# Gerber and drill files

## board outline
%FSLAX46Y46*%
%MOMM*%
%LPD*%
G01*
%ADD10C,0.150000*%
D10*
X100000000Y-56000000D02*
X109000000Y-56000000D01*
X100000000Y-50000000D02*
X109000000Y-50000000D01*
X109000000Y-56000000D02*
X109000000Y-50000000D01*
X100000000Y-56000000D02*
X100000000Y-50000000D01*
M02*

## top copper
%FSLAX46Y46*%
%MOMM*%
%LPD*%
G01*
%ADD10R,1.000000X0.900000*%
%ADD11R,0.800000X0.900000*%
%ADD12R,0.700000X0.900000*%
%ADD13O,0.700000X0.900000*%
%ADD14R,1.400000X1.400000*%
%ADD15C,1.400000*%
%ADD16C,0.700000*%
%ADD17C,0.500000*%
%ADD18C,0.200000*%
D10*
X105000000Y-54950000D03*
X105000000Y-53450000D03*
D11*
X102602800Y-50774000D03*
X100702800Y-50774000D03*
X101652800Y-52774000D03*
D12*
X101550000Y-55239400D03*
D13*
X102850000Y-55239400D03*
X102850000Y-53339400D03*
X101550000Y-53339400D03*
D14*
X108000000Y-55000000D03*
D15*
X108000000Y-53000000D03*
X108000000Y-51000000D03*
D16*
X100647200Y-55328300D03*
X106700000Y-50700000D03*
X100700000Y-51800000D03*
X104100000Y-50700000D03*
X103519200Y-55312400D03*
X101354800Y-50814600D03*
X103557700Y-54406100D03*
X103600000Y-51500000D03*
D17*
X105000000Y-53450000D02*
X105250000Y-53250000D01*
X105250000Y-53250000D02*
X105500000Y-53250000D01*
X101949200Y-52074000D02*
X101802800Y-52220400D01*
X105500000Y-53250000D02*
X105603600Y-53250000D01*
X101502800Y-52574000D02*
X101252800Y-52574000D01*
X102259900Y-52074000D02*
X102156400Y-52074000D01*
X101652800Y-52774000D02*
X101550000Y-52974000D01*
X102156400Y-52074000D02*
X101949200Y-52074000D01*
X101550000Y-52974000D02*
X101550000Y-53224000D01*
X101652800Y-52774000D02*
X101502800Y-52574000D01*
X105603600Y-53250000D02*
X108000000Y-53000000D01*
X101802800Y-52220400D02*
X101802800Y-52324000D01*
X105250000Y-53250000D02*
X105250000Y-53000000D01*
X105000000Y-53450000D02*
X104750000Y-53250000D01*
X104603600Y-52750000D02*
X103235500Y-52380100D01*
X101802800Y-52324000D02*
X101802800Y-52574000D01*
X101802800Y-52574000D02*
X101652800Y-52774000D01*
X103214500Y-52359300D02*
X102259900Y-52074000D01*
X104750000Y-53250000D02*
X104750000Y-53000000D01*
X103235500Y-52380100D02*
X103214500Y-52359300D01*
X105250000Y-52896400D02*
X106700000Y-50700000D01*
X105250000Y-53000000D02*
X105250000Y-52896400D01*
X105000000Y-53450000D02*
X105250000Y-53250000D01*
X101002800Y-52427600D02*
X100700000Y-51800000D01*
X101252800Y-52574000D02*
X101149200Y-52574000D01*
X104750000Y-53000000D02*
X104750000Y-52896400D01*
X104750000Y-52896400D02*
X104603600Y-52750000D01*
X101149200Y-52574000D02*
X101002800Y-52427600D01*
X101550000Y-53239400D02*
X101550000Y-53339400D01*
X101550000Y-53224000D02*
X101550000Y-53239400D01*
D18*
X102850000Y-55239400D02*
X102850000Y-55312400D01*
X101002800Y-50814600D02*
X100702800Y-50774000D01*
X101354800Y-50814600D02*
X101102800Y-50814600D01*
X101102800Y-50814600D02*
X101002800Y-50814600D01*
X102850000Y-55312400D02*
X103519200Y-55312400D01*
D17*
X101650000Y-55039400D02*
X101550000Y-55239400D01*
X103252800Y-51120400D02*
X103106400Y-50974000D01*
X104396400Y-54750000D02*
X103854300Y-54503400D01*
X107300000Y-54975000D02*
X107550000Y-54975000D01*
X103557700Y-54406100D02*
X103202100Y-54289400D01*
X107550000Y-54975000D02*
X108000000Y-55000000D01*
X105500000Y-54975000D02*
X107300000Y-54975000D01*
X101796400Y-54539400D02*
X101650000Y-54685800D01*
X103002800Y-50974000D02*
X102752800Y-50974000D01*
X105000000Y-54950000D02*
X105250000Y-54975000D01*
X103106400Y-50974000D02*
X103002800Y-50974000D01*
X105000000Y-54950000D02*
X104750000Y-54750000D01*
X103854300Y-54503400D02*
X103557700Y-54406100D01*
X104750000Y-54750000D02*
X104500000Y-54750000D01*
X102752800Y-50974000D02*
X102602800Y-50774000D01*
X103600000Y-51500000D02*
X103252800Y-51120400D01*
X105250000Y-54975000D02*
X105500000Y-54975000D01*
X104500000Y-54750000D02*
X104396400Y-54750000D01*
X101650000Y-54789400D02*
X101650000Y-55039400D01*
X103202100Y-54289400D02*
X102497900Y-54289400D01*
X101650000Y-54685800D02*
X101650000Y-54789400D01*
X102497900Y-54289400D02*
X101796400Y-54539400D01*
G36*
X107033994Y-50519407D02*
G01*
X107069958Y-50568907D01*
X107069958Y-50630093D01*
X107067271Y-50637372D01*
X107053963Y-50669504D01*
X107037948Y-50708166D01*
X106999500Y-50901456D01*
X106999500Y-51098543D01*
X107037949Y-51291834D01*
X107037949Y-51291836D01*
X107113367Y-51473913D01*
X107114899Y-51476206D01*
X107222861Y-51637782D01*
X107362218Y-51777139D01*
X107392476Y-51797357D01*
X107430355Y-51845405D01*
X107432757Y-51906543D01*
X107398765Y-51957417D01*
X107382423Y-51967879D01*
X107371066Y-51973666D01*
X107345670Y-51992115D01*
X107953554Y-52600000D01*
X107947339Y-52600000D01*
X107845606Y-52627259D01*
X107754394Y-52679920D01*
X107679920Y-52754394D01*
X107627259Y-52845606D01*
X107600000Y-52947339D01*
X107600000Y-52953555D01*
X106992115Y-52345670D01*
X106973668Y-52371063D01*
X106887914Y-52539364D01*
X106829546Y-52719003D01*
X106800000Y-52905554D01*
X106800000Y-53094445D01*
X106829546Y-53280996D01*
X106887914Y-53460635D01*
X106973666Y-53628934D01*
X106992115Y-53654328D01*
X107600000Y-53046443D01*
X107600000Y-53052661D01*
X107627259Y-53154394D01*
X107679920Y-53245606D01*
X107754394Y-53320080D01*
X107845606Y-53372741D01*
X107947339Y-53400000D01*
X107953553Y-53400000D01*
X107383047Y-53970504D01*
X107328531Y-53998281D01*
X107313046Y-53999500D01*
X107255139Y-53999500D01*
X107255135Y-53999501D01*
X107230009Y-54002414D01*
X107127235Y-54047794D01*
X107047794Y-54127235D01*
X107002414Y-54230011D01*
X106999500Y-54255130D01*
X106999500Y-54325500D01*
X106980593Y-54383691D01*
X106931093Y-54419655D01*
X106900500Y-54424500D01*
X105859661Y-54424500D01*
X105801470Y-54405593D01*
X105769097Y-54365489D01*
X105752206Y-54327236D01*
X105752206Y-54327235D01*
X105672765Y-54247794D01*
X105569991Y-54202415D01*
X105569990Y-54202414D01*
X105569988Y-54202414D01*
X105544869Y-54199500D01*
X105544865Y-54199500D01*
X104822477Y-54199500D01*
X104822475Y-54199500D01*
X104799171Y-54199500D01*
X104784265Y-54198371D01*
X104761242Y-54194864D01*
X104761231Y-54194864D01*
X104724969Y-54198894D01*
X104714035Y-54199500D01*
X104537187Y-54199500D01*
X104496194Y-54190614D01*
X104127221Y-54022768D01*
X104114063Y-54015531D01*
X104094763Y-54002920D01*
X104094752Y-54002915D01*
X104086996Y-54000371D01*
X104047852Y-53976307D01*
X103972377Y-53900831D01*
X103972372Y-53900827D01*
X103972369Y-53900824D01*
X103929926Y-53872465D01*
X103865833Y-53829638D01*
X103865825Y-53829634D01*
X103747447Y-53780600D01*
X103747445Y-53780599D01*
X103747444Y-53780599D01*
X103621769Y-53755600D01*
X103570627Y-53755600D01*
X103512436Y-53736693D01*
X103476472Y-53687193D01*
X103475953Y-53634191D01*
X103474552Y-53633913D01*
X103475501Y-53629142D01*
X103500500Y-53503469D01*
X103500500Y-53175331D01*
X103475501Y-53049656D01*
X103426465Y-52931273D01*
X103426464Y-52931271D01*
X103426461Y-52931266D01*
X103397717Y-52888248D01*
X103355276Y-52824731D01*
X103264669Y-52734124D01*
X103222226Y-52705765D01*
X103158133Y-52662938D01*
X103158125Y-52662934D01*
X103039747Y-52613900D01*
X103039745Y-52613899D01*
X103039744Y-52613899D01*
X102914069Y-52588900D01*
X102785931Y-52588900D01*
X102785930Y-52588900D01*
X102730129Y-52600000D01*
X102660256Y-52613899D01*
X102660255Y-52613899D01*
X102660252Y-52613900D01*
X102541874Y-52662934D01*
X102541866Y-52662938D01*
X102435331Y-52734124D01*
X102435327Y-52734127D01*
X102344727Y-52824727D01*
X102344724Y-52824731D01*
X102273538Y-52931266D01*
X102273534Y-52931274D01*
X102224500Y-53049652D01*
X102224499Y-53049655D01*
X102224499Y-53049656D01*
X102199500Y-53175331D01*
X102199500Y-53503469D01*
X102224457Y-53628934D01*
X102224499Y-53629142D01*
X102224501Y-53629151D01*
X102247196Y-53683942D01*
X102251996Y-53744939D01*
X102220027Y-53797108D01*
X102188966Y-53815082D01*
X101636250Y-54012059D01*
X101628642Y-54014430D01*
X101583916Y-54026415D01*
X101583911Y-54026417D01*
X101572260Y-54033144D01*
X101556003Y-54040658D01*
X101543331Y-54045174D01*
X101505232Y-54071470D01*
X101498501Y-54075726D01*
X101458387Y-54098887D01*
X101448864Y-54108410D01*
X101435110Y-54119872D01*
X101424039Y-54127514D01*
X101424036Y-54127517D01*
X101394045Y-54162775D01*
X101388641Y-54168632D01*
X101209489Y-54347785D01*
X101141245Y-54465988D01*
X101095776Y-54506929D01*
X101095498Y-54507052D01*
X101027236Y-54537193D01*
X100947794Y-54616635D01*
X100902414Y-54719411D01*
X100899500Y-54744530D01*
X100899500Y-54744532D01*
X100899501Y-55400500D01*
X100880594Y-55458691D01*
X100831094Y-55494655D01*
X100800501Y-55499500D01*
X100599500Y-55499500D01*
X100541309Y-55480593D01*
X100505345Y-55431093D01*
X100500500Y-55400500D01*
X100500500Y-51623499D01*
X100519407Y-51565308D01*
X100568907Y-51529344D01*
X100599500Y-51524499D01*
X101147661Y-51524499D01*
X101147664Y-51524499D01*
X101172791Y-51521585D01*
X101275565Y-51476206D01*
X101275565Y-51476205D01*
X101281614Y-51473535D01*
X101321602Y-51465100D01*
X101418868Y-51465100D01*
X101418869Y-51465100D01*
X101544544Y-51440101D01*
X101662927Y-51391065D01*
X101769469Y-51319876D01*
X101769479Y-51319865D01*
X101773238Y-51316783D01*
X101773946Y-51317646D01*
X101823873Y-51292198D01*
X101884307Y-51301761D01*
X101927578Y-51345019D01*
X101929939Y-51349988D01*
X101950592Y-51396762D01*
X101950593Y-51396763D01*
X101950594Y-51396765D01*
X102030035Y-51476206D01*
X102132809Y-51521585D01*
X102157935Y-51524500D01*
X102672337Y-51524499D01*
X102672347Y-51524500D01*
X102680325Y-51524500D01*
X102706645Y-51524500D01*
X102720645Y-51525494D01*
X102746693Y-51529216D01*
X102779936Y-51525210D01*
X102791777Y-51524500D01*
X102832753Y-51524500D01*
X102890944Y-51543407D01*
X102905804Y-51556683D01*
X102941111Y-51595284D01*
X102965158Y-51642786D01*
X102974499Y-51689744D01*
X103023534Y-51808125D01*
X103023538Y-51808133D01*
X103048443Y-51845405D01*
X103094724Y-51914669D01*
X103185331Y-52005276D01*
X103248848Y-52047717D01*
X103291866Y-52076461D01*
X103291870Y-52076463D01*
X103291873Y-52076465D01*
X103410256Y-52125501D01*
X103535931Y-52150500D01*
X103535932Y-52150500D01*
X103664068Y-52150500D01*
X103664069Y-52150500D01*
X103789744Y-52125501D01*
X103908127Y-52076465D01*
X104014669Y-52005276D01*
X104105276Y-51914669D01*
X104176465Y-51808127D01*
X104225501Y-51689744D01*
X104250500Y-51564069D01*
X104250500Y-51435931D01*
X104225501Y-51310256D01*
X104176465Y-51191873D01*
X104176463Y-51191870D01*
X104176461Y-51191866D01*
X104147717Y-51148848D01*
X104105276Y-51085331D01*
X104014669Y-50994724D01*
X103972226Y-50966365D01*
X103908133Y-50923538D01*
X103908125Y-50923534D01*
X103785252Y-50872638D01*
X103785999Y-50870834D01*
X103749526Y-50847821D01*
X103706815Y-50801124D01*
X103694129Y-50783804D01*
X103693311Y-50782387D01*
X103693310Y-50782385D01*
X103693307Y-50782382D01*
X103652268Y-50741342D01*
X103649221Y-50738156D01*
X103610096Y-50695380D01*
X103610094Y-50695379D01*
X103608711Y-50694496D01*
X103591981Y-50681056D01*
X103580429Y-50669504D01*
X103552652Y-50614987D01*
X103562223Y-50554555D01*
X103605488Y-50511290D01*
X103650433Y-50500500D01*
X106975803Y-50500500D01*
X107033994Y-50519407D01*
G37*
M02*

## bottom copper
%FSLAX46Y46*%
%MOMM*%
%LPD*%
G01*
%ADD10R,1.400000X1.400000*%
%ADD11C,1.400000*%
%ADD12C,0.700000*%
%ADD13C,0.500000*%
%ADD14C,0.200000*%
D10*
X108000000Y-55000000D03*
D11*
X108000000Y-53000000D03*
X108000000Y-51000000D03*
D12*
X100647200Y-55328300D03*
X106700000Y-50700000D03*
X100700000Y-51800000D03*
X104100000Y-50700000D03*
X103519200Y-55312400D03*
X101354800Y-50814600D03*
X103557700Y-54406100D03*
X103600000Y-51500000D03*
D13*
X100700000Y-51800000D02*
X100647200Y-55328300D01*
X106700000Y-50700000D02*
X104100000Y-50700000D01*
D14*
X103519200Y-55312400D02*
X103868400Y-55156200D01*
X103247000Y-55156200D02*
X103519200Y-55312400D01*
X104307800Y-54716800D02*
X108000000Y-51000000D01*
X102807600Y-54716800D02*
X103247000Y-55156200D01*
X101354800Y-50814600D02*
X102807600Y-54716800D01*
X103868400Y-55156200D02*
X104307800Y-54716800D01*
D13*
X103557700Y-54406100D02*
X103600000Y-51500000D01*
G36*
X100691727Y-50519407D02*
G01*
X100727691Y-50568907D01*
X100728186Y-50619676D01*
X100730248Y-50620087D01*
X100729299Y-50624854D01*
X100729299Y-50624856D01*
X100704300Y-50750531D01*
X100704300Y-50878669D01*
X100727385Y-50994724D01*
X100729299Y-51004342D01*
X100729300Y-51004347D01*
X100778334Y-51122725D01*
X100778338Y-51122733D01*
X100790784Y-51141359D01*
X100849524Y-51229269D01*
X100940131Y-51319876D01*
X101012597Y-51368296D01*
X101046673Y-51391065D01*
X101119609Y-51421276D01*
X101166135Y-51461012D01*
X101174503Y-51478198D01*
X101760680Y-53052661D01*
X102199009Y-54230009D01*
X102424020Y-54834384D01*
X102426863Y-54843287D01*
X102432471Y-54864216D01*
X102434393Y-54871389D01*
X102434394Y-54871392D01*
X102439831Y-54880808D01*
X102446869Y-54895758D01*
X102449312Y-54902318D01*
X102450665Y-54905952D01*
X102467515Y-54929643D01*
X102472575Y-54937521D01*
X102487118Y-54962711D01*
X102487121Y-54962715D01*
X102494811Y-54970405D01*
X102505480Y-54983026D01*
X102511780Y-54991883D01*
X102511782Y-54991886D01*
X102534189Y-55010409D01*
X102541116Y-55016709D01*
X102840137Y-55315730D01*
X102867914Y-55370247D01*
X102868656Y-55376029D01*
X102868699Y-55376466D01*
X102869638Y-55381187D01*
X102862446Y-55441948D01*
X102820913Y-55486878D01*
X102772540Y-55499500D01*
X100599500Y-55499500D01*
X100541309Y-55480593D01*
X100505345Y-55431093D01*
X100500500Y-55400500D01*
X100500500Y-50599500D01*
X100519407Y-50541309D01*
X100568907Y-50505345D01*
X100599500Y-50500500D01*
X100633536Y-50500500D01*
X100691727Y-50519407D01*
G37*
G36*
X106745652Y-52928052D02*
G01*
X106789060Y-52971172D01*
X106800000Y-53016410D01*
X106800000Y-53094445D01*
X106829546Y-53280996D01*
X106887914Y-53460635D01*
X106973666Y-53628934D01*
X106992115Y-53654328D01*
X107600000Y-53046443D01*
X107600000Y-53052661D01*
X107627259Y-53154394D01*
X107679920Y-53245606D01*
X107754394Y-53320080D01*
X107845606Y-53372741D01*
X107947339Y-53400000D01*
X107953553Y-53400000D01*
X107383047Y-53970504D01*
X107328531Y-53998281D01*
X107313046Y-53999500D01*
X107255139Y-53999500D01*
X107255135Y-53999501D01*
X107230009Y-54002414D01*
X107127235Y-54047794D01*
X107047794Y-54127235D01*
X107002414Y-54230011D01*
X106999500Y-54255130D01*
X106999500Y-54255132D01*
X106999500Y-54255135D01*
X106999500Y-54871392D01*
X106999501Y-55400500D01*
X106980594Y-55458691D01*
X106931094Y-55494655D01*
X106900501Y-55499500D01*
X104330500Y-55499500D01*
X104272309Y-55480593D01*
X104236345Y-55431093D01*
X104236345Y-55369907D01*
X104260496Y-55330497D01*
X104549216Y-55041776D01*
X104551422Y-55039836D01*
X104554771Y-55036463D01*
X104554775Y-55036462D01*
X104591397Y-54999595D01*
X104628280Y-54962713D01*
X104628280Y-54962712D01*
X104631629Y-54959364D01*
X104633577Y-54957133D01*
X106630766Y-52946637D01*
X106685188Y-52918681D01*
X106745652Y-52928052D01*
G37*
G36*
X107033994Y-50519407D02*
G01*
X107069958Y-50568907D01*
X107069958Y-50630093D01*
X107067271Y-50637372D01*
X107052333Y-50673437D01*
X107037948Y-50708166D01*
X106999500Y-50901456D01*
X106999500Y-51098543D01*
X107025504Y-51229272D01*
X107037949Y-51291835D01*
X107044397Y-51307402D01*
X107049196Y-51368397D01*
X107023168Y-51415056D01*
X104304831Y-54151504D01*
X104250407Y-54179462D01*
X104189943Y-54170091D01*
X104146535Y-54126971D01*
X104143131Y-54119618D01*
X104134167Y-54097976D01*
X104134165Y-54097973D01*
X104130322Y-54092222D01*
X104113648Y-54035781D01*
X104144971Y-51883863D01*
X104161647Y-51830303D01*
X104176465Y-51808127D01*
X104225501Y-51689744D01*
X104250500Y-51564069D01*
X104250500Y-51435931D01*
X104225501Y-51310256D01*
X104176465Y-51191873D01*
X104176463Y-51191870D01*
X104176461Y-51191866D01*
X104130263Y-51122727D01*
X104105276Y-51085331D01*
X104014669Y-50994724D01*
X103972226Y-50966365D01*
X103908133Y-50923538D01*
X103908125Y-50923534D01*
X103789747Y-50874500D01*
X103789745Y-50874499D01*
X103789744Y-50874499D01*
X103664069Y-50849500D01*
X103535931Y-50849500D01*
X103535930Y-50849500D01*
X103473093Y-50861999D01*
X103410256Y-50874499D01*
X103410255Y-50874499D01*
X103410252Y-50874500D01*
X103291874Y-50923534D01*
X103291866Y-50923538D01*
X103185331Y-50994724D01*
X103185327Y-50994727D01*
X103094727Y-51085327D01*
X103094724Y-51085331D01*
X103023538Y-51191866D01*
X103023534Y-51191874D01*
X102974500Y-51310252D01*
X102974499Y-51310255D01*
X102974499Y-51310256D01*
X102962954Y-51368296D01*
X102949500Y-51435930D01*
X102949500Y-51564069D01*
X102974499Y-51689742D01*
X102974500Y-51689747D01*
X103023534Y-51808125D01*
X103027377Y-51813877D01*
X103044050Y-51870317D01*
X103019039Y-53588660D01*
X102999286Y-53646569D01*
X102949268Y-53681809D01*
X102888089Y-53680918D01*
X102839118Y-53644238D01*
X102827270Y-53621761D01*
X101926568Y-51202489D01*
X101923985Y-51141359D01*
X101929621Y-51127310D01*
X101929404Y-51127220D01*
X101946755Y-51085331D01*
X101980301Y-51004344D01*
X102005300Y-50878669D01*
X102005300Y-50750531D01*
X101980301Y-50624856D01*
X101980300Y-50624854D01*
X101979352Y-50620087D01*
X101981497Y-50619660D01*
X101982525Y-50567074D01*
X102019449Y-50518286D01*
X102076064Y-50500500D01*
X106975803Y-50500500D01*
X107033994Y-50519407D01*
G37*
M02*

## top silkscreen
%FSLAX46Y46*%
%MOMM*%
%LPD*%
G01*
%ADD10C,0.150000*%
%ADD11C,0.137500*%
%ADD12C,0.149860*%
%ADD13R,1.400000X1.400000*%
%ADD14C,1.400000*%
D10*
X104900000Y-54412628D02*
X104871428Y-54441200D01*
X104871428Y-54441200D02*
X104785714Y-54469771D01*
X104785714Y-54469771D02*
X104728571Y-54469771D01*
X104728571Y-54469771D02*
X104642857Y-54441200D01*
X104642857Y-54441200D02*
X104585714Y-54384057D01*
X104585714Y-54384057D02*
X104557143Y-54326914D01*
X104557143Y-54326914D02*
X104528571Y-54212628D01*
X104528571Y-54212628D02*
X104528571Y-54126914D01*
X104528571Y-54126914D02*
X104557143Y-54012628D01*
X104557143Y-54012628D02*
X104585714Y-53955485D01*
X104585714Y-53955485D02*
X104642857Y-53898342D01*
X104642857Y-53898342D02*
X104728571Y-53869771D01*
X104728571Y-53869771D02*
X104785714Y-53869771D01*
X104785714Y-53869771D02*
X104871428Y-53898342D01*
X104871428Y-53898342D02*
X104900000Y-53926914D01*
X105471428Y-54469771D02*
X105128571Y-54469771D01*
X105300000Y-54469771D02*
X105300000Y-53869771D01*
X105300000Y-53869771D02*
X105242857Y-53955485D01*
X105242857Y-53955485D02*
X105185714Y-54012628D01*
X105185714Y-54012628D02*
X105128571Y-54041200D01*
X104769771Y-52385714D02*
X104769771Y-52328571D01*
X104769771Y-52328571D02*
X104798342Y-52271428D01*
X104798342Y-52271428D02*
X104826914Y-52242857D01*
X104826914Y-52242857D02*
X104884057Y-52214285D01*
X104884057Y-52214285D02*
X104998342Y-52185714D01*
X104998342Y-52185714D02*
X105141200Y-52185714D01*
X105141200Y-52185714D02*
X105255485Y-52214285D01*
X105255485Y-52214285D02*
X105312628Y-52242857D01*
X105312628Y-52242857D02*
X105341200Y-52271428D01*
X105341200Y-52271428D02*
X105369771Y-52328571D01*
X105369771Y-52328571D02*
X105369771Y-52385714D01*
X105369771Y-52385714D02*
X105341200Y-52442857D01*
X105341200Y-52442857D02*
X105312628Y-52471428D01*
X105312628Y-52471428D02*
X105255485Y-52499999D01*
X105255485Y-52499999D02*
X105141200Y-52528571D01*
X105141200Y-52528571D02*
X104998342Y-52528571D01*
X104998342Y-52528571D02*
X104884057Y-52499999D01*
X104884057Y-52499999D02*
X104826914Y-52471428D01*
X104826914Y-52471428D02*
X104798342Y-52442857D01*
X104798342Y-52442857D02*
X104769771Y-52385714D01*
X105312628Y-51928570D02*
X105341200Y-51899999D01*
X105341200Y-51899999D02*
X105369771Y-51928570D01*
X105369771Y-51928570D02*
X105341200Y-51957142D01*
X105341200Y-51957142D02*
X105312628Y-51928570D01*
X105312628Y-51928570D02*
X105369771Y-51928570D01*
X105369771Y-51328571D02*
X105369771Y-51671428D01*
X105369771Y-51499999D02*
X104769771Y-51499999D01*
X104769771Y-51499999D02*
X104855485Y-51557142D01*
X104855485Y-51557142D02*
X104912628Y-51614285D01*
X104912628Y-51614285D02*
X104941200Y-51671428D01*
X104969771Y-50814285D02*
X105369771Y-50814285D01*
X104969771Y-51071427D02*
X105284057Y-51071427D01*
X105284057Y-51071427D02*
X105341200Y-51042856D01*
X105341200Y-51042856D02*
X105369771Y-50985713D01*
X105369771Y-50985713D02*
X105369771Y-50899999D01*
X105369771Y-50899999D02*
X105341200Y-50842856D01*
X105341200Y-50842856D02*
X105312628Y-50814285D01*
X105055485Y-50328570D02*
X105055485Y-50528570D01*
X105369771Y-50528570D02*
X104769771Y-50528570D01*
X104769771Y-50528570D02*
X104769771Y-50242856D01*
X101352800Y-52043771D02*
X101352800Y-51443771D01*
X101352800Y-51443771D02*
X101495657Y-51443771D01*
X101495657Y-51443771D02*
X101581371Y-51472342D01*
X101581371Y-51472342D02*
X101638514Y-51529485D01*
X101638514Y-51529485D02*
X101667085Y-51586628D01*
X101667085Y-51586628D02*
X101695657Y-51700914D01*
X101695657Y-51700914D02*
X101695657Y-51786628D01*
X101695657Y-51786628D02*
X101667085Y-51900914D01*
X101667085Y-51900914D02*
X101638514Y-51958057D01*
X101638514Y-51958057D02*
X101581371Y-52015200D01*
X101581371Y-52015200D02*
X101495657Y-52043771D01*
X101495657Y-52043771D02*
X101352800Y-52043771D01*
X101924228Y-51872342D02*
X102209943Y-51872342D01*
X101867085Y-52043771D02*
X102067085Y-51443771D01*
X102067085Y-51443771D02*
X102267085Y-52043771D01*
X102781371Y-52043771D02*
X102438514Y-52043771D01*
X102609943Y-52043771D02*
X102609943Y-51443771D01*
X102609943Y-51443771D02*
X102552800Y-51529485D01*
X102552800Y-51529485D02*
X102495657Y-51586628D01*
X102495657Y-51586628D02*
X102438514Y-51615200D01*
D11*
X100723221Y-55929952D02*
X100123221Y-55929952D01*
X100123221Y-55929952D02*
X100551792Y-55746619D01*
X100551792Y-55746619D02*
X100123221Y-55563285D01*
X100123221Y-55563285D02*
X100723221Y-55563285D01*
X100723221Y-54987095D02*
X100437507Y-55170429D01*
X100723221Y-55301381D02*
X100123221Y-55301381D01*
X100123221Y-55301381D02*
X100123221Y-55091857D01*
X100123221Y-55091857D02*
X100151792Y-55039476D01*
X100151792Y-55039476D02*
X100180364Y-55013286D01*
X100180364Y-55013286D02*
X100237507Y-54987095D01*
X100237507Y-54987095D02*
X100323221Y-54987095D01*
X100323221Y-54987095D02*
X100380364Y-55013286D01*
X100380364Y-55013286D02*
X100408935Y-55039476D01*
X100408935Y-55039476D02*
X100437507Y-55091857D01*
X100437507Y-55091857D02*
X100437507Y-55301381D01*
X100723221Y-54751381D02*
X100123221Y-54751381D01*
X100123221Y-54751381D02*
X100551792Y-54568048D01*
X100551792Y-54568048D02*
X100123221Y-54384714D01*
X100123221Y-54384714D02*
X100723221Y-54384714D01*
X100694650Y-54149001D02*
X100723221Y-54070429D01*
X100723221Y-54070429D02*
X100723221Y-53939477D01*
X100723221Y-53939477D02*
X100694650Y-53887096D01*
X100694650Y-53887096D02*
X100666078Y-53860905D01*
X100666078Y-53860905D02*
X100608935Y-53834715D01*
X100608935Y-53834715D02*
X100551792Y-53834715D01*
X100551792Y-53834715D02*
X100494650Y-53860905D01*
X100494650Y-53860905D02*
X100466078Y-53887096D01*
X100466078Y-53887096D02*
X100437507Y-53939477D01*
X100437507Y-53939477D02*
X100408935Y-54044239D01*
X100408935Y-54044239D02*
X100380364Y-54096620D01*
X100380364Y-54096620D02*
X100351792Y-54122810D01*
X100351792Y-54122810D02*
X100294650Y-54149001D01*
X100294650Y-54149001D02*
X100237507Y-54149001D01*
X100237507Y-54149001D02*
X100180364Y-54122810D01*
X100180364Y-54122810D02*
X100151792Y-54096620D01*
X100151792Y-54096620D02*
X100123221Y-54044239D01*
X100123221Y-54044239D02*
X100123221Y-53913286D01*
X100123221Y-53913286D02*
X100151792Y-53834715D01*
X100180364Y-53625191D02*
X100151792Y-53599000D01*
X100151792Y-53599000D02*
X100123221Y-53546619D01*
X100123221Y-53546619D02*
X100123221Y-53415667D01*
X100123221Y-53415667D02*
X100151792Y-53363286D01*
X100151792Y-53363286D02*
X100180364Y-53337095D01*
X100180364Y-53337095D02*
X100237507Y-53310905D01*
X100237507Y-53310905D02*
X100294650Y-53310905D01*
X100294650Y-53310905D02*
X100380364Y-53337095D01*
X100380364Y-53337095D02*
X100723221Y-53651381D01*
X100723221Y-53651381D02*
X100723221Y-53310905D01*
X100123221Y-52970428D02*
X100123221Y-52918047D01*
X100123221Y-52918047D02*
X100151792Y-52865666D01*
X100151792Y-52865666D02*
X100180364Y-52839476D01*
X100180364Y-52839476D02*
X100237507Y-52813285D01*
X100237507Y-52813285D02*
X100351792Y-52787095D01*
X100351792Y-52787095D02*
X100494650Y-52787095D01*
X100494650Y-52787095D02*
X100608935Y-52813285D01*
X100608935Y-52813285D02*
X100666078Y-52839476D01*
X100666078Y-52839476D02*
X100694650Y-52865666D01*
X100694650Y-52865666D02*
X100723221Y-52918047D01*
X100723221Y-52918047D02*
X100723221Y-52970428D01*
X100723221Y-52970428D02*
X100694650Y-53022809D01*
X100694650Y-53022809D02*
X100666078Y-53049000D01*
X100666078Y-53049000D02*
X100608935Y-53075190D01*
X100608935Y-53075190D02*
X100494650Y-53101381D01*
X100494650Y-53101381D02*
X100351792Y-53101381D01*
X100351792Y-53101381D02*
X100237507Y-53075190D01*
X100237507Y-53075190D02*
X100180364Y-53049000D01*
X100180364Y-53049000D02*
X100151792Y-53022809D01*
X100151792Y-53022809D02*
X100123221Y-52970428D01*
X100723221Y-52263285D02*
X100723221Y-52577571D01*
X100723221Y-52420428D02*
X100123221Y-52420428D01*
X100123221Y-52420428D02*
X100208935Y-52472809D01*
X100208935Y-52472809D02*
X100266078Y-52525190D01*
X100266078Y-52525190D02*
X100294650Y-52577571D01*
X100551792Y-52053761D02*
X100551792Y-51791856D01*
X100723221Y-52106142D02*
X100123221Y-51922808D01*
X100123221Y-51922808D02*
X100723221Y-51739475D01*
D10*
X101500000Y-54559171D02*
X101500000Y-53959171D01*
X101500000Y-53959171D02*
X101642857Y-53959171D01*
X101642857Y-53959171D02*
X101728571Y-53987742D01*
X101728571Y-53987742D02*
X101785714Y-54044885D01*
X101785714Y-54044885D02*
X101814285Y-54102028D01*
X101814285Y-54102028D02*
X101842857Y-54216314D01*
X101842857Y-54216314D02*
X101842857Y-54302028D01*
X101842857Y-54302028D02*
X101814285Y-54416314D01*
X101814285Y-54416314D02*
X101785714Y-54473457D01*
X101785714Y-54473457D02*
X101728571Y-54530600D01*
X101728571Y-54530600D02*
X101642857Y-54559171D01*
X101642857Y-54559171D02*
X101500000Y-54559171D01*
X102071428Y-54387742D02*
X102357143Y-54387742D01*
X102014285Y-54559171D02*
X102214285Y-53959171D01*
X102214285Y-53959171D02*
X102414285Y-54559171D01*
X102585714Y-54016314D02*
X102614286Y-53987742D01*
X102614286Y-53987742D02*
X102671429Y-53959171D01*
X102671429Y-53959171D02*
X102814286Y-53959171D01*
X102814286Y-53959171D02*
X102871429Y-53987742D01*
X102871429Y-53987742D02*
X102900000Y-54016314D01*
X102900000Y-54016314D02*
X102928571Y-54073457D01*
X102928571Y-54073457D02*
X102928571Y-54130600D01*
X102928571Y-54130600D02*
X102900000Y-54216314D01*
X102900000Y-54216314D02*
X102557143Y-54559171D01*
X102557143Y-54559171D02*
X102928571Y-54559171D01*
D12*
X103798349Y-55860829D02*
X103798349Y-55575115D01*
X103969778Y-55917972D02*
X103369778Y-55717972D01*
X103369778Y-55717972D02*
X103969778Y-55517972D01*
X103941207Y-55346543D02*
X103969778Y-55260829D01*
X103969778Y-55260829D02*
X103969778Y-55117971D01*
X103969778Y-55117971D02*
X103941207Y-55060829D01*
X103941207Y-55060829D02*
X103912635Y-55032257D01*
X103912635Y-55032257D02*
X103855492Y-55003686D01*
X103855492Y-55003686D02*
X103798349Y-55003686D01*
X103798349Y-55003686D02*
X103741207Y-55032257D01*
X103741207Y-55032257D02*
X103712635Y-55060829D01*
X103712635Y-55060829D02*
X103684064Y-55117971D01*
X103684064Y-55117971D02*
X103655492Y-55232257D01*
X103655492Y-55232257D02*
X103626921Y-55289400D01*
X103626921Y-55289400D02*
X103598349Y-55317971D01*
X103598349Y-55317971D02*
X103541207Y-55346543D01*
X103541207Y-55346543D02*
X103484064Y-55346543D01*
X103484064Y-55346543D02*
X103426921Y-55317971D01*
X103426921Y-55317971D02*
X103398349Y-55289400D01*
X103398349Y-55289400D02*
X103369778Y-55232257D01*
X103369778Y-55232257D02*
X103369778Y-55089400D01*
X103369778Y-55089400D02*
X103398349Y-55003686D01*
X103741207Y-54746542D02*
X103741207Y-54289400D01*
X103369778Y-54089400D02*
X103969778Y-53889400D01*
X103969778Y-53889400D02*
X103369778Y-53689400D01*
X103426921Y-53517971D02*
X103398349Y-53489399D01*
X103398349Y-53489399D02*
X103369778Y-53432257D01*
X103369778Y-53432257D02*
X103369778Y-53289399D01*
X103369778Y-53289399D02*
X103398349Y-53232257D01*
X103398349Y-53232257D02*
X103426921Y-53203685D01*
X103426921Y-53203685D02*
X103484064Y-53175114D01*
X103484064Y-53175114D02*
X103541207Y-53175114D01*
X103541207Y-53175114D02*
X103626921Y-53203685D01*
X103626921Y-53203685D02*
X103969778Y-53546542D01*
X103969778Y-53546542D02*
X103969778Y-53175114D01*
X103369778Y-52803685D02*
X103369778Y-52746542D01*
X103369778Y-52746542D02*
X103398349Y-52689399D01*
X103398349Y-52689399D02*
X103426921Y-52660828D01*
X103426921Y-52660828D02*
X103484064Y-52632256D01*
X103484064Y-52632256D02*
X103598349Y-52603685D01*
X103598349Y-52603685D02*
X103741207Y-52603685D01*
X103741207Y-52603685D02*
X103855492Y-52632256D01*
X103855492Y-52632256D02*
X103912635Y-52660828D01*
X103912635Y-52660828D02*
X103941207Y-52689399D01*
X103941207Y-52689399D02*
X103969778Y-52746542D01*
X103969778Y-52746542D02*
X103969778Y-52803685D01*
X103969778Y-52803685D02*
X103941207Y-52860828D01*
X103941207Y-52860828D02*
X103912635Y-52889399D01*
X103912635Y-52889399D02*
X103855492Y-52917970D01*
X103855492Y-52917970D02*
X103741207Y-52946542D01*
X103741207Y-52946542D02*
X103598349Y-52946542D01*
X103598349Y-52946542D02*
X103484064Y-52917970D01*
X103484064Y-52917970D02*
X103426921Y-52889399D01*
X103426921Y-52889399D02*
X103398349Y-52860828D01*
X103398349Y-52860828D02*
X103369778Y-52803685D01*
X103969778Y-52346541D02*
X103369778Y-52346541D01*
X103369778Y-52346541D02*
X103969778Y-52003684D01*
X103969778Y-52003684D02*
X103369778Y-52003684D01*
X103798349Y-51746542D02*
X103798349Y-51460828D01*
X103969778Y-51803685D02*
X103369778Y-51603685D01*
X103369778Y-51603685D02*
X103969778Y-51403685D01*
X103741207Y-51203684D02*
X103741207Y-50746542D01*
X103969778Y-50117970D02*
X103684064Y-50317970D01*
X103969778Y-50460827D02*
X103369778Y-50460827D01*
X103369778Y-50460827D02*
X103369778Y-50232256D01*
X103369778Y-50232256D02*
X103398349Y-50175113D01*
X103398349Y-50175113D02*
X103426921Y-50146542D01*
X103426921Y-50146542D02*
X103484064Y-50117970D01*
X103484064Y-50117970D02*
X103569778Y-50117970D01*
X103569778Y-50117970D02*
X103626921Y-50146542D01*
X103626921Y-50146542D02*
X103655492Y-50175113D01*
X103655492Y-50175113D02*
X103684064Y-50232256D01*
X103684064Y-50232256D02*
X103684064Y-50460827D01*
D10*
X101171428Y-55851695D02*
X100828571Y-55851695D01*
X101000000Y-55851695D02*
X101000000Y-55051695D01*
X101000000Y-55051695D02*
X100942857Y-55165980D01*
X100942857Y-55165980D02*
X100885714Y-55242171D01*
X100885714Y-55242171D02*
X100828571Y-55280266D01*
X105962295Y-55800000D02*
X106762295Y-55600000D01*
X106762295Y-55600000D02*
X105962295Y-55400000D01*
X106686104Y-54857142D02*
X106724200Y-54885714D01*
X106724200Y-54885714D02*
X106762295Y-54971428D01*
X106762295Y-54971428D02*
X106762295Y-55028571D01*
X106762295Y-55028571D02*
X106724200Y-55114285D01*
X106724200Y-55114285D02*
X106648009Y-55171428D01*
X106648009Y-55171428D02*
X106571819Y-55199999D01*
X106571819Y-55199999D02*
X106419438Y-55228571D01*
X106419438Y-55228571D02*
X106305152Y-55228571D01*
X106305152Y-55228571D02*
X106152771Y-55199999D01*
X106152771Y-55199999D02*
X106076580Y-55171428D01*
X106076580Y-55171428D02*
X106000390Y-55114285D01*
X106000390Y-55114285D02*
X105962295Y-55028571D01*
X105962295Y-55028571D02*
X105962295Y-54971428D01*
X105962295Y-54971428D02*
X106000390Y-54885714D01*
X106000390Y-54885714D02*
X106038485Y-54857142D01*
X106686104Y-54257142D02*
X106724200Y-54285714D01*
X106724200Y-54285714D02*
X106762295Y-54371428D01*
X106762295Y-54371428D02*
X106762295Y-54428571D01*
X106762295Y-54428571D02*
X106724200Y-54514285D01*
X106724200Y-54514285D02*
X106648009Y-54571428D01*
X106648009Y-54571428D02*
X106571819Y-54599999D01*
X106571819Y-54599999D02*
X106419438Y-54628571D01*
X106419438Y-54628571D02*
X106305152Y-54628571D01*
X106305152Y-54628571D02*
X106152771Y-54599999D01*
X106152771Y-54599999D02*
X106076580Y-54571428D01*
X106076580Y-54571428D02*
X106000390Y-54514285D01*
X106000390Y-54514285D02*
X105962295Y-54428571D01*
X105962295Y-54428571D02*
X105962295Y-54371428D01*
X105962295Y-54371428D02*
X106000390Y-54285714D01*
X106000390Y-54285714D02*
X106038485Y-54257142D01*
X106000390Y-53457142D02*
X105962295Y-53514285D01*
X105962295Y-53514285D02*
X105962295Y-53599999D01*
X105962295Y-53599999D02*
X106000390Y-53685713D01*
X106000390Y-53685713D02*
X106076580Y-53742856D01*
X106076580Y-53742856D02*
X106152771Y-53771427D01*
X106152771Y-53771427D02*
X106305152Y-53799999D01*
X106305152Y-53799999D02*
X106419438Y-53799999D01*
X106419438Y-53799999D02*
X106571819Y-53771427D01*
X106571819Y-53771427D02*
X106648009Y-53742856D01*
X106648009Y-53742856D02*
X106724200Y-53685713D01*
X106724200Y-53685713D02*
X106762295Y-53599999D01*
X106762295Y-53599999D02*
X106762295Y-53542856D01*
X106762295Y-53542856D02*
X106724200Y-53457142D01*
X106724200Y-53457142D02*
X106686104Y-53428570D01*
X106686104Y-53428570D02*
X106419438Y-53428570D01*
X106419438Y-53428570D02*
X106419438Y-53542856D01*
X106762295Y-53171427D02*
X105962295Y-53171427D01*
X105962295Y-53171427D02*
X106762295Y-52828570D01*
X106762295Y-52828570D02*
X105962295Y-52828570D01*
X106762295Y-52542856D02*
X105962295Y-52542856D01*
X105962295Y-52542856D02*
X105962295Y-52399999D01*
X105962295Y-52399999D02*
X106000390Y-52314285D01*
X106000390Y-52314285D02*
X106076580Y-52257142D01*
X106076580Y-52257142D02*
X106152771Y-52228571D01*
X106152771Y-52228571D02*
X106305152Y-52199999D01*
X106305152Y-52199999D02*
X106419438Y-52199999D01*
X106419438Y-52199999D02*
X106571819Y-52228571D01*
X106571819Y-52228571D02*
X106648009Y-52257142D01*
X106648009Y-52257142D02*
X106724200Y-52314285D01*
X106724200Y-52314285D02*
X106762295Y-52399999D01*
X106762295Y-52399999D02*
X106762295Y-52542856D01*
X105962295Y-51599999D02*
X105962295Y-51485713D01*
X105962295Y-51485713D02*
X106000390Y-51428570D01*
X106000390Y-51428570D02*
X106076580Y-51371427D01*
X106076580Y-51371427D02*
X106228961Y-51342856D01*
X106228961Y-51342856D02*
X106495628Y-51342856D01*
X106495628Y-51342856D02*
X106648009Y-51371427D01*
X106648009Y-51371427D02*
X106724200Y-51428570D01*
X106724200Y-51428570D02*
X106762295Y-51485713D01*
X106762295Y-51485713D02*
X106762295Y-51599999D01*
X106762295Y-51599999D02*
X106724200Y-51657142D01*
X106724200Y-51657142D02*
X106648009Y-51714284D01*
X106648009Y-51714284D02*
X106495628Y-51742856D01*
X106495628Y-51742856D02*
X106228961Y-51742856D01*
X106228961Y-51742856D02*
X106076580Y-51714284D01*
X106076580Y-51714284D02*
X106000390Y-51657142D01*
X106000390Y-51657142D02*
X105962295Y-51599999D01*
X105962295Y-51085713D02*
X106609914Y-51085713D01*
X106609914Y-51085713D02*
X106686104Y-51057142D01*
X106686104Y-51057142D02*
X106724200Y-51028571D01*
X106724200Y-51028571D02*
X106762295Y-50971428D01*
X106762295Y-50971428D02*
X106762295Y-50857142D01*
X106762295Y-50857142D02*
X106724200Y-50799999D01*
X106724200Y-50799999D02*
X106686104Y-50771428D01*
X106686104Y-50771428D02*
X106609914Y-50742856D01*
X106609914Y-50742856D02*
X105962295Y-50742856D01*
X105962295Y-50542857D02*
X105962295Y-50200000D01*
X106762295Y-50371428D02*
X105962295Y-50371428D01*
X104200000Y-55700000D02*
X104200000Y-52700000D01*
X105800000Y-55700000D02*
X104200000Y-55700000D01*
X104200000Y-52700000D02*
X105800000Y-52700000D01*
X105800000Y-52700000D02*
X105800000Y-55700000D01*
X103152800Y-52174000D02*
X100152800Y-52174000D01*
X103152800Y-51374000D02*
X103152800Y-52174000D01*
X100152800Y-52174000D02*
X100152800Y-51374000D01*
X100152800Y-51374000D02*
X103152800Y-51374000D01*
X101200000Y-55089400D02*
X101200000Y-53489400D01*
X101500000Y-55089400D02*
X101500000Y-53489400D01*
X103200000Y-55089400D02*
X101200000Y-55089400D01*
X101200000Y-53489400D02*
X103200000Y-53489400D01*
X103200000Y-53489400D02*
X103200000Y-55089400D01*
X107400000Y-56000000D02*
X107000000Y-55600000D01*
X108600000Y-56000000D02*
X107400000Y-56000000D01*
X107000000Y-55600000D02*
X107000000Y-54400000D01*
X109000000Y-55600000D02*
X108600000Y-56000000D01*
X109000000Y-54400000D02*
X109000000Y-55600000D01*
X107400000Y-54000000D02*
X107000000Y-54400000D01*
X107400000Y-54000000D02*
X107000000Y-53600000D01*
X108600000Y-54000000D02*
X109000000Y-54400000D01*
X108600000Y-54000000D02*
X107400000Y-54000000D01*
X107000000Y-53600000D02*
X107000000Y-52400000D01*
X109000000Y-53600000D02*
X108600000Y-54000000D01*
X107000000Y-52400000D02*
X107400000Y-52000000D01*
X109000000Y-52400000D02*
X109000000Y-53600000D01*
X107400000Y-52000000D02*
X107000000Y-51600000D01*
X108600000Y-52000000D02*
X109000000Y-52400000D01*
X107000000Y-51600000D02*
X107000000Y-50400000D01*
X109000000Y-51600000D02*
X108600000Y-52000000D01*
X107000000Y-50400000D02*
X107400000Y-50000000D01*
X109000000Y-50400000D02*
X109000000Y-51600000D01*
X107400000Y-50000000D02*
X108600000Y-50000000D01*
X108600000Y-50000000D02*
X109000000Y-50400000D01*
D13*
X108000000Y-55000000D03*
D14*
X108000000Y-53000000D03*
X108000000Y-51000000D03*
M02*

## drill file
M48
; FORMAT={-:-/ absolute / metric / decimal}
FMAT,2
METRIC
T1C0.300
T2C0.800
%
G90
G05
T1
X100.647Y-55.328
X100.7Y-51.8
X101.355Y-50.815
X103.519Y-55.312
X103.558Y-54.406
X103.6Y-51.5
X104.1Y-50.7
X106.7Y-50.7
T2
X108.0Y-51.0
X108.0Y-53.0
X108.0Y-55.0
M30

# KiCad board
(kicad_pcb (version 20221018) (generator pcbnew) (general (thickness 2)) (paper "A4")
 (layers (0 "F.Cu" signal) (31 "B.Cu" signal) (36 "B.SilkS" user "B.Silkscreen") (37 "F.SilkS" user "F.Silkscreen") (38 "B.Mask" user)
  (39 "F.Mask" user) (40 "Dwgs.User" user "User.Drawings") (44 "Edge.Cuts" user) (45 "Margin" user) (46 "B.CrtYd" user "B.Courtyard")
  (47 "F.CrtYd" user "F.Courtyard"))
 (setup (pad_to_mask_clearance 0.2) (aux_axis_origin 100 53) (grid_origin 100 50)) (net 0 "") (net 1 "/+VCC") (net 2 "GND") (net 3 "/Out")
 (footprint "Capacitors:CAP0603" (layer "F.Cu") (at 105 54.2 90)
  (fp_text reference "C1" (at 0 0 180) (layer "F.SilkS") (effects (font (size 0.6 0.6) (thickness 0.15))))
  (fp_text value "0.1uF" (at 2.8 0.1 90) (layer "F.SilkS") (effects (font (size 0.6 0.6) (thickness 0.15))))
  (fp_line (start -1.5 -0.8) (end 1.5 -0.8) (stroke (width 0.15) (type solid)) (layer "F.SilkS"))
  (fp_line (start -1.5 0.8) (end -1.5 -0.8) (stroke (width 0.15) (type solid)) (layer "F.SilkS"))
  (fp_line (start 1.5 -0.8) (end 1.5 0.8) (stroke (width 0.15) (type solid)) (layer "F.SilkS"))
  (fp_line (start 1.5 0.8) (end -1.5 0.8) (stroke (width 0.15) (type solid)) (layer "F.SilkS"))
  (pad "1" smd rect (at -0.75 0 90) (size 0.9 1) (layers "F.Cu" "F.Paste" "F.Mask") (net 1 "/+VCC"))
  (pad "2" smd rect (at 0.75 0 90) (size 0.9 1) (layers "F.Cu" "F.Paste" "F.Mask") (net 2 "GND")))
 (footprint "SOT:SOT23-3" (layer "F.Cu") (at 101.6528 51.774 180)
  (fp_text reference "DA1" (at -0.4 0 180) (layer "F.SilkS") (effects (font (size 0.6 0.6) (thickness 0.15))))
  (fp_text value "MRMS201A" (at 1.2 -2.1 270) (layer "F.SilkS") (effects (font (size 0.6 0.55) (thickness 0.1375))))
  (fp_line (start -1.5 -0.4) (end 1.5 -0.4) (stroke (width 0.15) (type solid)) (layer "F.SilkS"))
  (fp_line (start -1.5 0.4) (end -1.5 -0.4) (stroke (width 0.15) (type solid)) (layer "F.SilkS"))
  (fp_line (start 1.5 -0.4) (end 1.5 0.4) (stroke (width 0.15) (type solid)) (layer "F.SilkS"))
  (fp_line (start 1.5 0.4) (end -1.5 0.4) (stroke (width 0.15) (type solid)) (layer "F.SilkS"))
  (pad "1" smd rect (at -0.95 1 180) (size 0.8 0.9) (layers "F.Cu" "F.Paste" "F.Mask") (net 1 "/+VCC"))
  (pad "2" smd rect (at 0.95 1 180) (size 0.8 0.9) (layers "F.Cu" "F.Paste" "F.Mask") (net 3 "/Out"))
  (pad "3" smd rect (at 0 -1 180) (size 0.8 0.9) (layers "F.Cu" "F.Paste" "F.Mask") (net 2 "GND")))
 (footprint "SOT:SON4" (layer "F.Cu") (at 102.2 54.2894 90)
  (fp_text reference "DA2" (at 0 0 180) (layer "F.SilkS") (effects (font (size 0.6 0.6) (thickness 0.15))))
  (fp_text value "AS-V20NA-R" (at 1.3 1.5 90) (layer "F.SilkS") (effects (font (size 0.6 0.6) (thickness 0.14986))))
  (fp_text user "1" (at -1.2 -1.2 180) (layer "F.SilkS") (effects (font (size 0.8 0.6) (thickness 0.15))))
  (fp_line (start -0.8 -1) (end 0.8 -1) (stroke (width 0.15) (type solid)) (layer "F.SilkS"))
  (fp_line (start -0.8 -0.7) (end 0.8 -0.7) (stroke (width 0.15) (type solid)) (layer "F.SilkS"))
  (fp_line (start -0.8 1) (end -0.8 -1) (stroke (width 0.15) (type solid)) (layer "F.SilkS"))
  (fp_line (start 0.8 -1) (end 0.8 1) (stroke (width 0.15) (type solid)) (layer "F.SilkS"))
  (fp_line (start 0.8 1) (end -0.8 1) (stroke (width 0.15) (type solid)) (layer "F.SilkS"))
  (pad "1" smd rect (at -0.95 -0.65 90) (size 0.9 0.7) (layers "F.Cu" "F.Mask") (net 1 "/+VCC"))
  (pad "2" smd oval (at -0.95 0.65 90) (size 0.9 0.7) (layers "F.Cu" "F.Mask") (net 3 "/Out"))
  (pad "3" smd oval (at 0.95 0.65 90) (size 0.9 0.7) (layers "F.Cu" "F.Mask"))
  (pad "4" smd oval (at 0.95 -0.65 90) (size 0.9 0.7) (layers "F.Cu" "F.Mask") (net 2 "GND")))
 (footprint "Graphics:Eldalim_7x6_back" (layer "F.Cu") (at 103.5 52.9)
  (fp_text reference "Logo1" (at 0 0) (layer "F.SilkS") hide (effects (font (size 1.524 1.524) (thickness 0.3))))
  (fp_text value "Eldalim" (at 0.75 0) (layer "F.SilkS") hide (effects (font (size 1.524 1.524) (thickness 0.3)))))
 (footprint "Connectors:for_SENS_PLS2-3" (layer "F.Cu") (at 108 55 90)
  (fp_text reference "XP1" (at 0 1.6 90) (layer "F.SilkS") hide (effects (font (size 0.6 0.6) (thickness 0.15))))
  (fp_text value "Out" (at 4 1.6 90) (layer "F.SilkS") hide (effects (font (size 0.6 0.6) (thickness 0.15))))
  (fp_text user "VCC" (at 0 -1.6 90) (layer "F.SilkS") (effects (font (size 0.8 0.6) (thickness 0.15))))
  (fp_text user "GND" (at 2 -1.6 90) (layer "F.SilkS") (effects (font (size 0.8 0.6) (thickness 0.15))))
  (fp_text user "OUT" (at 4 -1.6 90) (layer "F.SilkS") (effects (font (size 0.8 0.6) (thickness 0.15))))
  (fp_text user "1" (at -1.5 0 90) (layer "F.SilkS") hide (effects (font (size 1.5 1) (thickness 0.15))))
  (fp_line (start -1 -0.6) (end -0.6 -1) (stroke (width 0.15) (type solid)) (layer "F.SilkS"))
  (fp_line (start -1 0.6) (end -1 -0.6) (stroke (width 0.15) (type solid)) (layer "F.SilkS"))
  (fp_line (start -0.6 -1) (end 0.6 -1) (stroke (width 0.15) (type solid)) (layer "F.SilkS"))
  (fp_line (start -0.6 1) (end -1 0.6) (stroke (width 0.15) (type solid)) (layer "F.SilkS"))
  (fp_line (start 0.6 1) (end -0.6 1) (stroke (width 0.15) (type solid)) (layer "F.SilkS"))
  (fp_line (start 1 -0.6) (end 0.6 -1) (stroke (width 0.15) (type solid)) (layer "F.SilkS"))
  (fp_line (start 1 -0.6) (end 1.4 -1) (stroke (width 0.15) (type solid)) (layer "F.SilkS"))
  (fp_line (start 1 0.6) (end 0.6 1) (stroke (width 0.15) (type solid)) (layer "F.SilkS"))
  (fp_line (start 1 0.6) (end 1 -0.6) (stroke (width 0.15) (type solid)) (layer "F.SilkS"))
  (fp_line (start 1.4 -1) (end 2.6 -1) (stroke (width 0.15) (type solid)) (layer "F.SilkS"))
  (fp_line (start 1.4 1) (end 1 0.6) (stroke (width 0.15) (type solid)) (layer "F.SilkS"))
  (fp_line (start 2.6 -1) (end 3 -0.6) (stroke (width 0.15) (type solid)) (layer "F.SilkS"))
  (fp_line (start 2.6 1) (end 1.4 1) (stroke (width 0.15) (type solid)) (layer "F.SilkS"))
  (fp_line (start 3 -0.6) (end 3.4 -1) (stroke (width 0.15) (type solid)) (layer "F.SilkS"))
  (fp_line (start 3 0.6) (end 2.6 1) (stroke (width 0.15) (type solid)) (layer "F.SilkS"))
  (fp_line (start 3.4 -1) (end 4.6 -1) (stroke (width 0.15) (type solid)) (layer "F.SilkS"))
  (fp_line (start 3.4 1) (end 3 0.6) (stroke (width 0.15) (type solid)) (layer "F.SilkS"))
  (fp_line (start 4.6 -1) (end 5 -0.6) (stroke (width 0.15) (type solid)) (layer "F.SilkS"))
  (fp_line (start 4.6 1) (end 3.4 1) (stroke (width 0.15) (type solid)) (layer "F.SilkS"))
  (fp_line (start 5 -0.6) (end 5 0.6) (stroke (width 0.15) (type solid)) (layer "F.SilkS"))
  (fp_line (start 5 0.6) (end 4.6 1) (stroke (width 0.15) (type solid)) (layer "F.SilkS"))
  (pad "1" thru_hole rect (at 0 0 90) (size 1.4 1.4) (drill 0.8) (layers "*.Cu" "*.Mask" "F.SilkS") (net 1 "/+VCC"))
  (pad "2" thru_hole circle (at 2 0 90) (size 1.4 1.4) (drill 0.8) (layers "*.Cu" "*.Mask" "F.SilkS") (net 2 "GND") (zone_connect 1))
  (pad "3" thru_hole circle (at 4 0 90) (size 1.4 1.4) (drill 0.8) (layers "*.Cu" "*.Mask" "F.SilkS") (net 3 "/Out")))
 (gr_line (start 100 56) (end 109 56) (stroke (width 0.15) (type solid)) (layer "Edge.Cuts"))
 (gr_line (start 100 50) (end 109 50) (stroke (width 0.15) (type solid)) (layer "Edge.Cuts"))
 (gr_line (start 109 56) (end 109 50) (stroke (width 0.15) (type solid)) (layer "Edge.Cuts"))
 (gr_line (start 100 56) (end 100 50) (stroke (width 0.15) (type solid)) (layer "Edge.Cuts"))
 (segment (start 105 53.45) (end 105.25 53.25) (width 0.5) (layer "F.Cu") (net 2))
 (segment (start 105.25 53.25) (end 105.5 53.25) (width 0.5) (layer "F.Cu") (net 2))
 (segment (start 101.9492 52.074) (end 101.8028 52.2204) (width 0.5) (layer "F.Cu") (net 2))
 (segment (start 105.5 53.25) (end 105.6036 53.25) (width 0.5) (layer "F.Cu") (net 2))
 (segment (start 101.5028 52.574) (end 101.2528 52.574) (width 0.5) (layer "F.Cu") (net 2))
 (segment (start 102.2599 52.074) (end 102.1564 52.074) (width 0.5) (layer "F.Cu") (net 2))
 (segment (start 101.6528 52.774) (end 101.55 52.974) (width 0.5) (layer "F.Cu") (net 2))
 (segment (start 102.1564 52.074) (end 101.9492 52.074) (width 0.5) (layer "F.Cu") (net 2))
 (segment (start 101.55 52.974) (end 101.55 53.224) (width 0.5) (layer "F.Cu") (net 2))
 (segment (start 101.6528 52.774) (end 101.5028 52.574) (width 0.5) (layer "F.Cu") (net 2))
 (segment (start 105.6036 53.25) (end 108 53) (width 0.5) (layer "F.Cu") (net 2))
 (segment (start 101.8028 52.2204) (end 101.8028 52.324) (width 0.5) (layer "F.Cu") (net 2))
 (segment (start 105.25 53.25) (end 105.25 53) (width 0.5) (layer "F.Cu") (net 2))
 (segment (start 105 53.45) (end 104.75 53.25) (width 0.5) (layer "F.Cu") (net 2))
 (segment (start 104.6036 52.75) (end 103.2355 52.3801) (width 0.5) (layer "F.Cu") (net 2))
 (segment (start 101.8028 52.324) (end 101.8028 52.574) (width 0.5) (layer "F.Cu") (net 2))
 (segment (start 101.8028 52.574) (end 101.6528 52.774) (width 0.5) (layer "F.Cu") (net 2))
 (segment (start 103.2145 52.3593) (end 102.2599 52.074) (width 0.5) (layer "F.Cu") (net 2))
 (segment (start 104.75 53.25) (end 104.75 53) (width 0.5) (layer "F.Cu") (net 2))
 (segment (start 103.2355 52.3801) (end 103.2145 52.3593) (width 0.5) (layer "F.Cu") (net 2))
 (segment (start 105.25 52.8964) (end 106.7 50.7) (width 0.5) (layer "F.Cu") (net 2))
 (segment (start 105.25 53) (end 105.25 52.8964) (width 0.5) (layer "F.Cu") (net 2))
 (segment (start 105 53.45) (end 105.25 53.25) (width 0.5) (layer "F.Cu") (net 2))
 (segment (start 101.0028 52.4276) (end 100.7 51.8) (width 0.5) (layer "F.Cu") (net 2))
 (segment (start 101.2528 52.574) (end 101.1492 52.574) (width 0.5) (layer "F.Cu") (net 2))
 (segment (start 104.75 53) (end 104.75 52.8964) (width 0.5) (layer "F.Cu") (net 2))
 (segment (start 104.75 52.8964) (end 104.6036 52.75) (width 0.5) (layer "F.Cu") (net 2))
 (segment (start 101.1492 52.574) (end 101.0028 52.4276) (width 0.5) (layer "F.Cu") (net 2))
 (segment (start 101.55 53.2394) (end 101.55 53.3394) (width 0.5) (layer "F.Cu") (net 2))
 (segment (start 101.55 53.224) (end 101.55 53.2394) (width 0.5) (layer "F.Cu") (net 2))
 (via (at 100.6472 55.3283) (size 0.7) (drill 0.3) (layers "F.Cu" "B.Cu") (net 2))
 (via (at 106.7 50.7) (size 0.7) (drill 0.3) (layers "F.Cu" "B.Cu") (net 2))
 (via (at 100.7 51.8) (size 0.7) (drill 0.3) (layers "F.Cu" "B.Cu") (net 2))
 (via (at 104.1 50.7) (size 0.7) (drill 0.3) (layers "F.Cu" "B.Cu") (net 2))
 (segment (start 100.7 51.8) (end 100.6472 55.3283) (width 0.5) (layer "B.Cu") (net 2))
 (segment (start 106.7 50.7) (end 104.1 50.7) (width 0.5) (layer "B.Cu") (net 2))
 (segment (start 102.85 55.2394) (end 102.85 55.3124) (width 0.2) (layer "F.Cu") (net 3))
 (segment (start 101.0028 50.8146) (end 100.7028 50.774) (width 0.2) (layer "F.Cu") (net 3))
 (segment (start 101.3548 50.8146) (end 101.1028 50.8146) (width 0.2) (layer "F.Cu") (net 3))
 (segment (start 101.1028 50.8146) (end 101.0028 50.8146) (width 0.2) (layer "F.Cu") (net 3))
 (segment (start 102.85 55.3124) (end 103.5192 55.3124) (width 0.2) (layer "F.Cu") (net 3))
 (via (at 103.5192 55.3124) (size 0.7) (drill 0.3) (layers "F.Cu" "B.Cu") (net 3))
 (via (at 101.3548 50.8146) (size 0.7) (drill 0.3) (layers "F.Cu" "B.Cu") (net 3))
 (segment (start 103.5192 55.3124) (end 103.8684 55.1562) (width 0.2) (layer "B.Cu") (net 3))
 (segment (start 103.247 55.1562) (end 103.5192 55.3124) (width 0.2) (layer "B.Cu") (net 3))
 (segment (start 104.3078 54.7168) (end 108 51) (width 0.2) (layer "B.Cu") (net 3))
 (segment (start 102.8076 54.7168) (end 103.247 55.1562) (width 0.2) (layer "B.Cu") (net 3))
 (segment (start 101.3548 50.8146) (end 102.8076 54.7168) (width 0.2) (layer "B.Cu") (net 3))
 (segment (start 103.8684 55.1562) (end 104.3078 54.7168) (width 0.2) (layer "B.Cu") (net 3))
 (segment (start 101.65 55.0394) (end 101.55 55.2394) (width 0.5) (layer "F.Cu") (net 1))
 (segment (start 103.2528 51.1204) (end 103.1064 50.974) (width 0.5) (layer "F.Cu") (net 1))
 (segment (start 104.3964 54.75) (end 103.8543 54.5034) (width 0.5) (layer "F.Cu") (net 1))
 (segment (start 107.3 54.975) (end 107.55 54.975) (width 0.5) (layer "F.Cu") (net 1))
 (segment (start 103.5577 54.4061) (end 103.2021 54.2894) (width 0.5) (layer "F.Cu") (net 1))
 (segment (start 107.55 54.975) (end 108 55) (width 0.5) (layer "F.Cu") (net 1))
 (segment (start 105.5 54.975) (end 107.3 54.975) (width 0.5) (layer "F.Cu") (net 1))
 (segment (start 101.7964 54.5394) (end 101.65 54.6858) (width 0.5) (layer "F.Cu") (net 1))
 (segment (start 103.0028 50.974) (end 102.7528 50.974) (width 0.5) (layer "F.Cu") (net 1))
 (segment (start 105 54.95) (end 105.25 54.975) (width 0.5) (layer "F.Cu") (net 1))
 (segment (start 103.1064 50.974) (end 103.0028 50.974) (width 0.5) (layer "F.Cu") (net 1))
 (segment (start 105 54.95) (end 104.75 54.75) (width 0.5) (layer "F.Cu") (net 1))
 (segment (start 103.8543 54.5034) (end 103.5577 54.4061) (width 0.5) (layer "F.Cu") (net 1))
 (segment (start 104.75 54.75) (end 104.5 54.75) (width 0.5) (layer "F.Cu") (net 1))
 (segment (start 102.7528 50.974) (end 102.6028 50.774) (width 0.5) (layer "F.Cu") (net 1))
 (segment (start 103.6 51.5) (end 103.2528 51.1204) (width 0.5) (layer "F.Cu") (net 1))
 (segment (start 105.25 54.975) (end 105.5 54.975) (width 0.5) (layer "F.Cu") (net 1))
 (segment (start 104.5 54.75) (end 104.3964 54.75) (width 0.5) (layer "F.Cu") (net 1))
 (segment (start 101.65 54.7894) (end 101.65 55.0394) (width 0.5) (layer "F.Cu") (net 1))
 (segment (start 103.2021 54.2894) (end 102.4979 54.2894) (width 0.5) (layer "F.Cu") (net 1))
 (segment (start 101.65 54.6858) (end 101.65 54.7894) (width 0.5) (layer "F.Cu") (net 1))
 (segment (start 102.4979 54.2894) (end 101.7964 54.5394) (width 0.5) (layer "F.Cu") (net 1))
 (via (at 103.5577 54.4061) (size 0.7) (drill 0.3) (layers "F.Cu" "B.Cu") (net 1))
 (via (at 103.6 51.5) (size 0.7) (drill 0.3) (layers "F.Cu" "B.Cu") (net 1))
 (segment (start 103.5577 54.4061) (end 103.6 51.5) (width 0.5) (layer "B.Cu") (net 1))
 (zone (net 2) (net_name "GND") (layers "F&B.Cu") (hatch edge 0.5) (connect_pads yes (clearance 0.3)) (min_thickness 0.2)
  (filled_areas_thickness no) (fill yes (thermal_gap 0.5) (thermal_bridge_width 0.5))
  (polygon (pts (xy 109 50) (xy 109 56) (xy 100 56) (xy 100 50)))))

